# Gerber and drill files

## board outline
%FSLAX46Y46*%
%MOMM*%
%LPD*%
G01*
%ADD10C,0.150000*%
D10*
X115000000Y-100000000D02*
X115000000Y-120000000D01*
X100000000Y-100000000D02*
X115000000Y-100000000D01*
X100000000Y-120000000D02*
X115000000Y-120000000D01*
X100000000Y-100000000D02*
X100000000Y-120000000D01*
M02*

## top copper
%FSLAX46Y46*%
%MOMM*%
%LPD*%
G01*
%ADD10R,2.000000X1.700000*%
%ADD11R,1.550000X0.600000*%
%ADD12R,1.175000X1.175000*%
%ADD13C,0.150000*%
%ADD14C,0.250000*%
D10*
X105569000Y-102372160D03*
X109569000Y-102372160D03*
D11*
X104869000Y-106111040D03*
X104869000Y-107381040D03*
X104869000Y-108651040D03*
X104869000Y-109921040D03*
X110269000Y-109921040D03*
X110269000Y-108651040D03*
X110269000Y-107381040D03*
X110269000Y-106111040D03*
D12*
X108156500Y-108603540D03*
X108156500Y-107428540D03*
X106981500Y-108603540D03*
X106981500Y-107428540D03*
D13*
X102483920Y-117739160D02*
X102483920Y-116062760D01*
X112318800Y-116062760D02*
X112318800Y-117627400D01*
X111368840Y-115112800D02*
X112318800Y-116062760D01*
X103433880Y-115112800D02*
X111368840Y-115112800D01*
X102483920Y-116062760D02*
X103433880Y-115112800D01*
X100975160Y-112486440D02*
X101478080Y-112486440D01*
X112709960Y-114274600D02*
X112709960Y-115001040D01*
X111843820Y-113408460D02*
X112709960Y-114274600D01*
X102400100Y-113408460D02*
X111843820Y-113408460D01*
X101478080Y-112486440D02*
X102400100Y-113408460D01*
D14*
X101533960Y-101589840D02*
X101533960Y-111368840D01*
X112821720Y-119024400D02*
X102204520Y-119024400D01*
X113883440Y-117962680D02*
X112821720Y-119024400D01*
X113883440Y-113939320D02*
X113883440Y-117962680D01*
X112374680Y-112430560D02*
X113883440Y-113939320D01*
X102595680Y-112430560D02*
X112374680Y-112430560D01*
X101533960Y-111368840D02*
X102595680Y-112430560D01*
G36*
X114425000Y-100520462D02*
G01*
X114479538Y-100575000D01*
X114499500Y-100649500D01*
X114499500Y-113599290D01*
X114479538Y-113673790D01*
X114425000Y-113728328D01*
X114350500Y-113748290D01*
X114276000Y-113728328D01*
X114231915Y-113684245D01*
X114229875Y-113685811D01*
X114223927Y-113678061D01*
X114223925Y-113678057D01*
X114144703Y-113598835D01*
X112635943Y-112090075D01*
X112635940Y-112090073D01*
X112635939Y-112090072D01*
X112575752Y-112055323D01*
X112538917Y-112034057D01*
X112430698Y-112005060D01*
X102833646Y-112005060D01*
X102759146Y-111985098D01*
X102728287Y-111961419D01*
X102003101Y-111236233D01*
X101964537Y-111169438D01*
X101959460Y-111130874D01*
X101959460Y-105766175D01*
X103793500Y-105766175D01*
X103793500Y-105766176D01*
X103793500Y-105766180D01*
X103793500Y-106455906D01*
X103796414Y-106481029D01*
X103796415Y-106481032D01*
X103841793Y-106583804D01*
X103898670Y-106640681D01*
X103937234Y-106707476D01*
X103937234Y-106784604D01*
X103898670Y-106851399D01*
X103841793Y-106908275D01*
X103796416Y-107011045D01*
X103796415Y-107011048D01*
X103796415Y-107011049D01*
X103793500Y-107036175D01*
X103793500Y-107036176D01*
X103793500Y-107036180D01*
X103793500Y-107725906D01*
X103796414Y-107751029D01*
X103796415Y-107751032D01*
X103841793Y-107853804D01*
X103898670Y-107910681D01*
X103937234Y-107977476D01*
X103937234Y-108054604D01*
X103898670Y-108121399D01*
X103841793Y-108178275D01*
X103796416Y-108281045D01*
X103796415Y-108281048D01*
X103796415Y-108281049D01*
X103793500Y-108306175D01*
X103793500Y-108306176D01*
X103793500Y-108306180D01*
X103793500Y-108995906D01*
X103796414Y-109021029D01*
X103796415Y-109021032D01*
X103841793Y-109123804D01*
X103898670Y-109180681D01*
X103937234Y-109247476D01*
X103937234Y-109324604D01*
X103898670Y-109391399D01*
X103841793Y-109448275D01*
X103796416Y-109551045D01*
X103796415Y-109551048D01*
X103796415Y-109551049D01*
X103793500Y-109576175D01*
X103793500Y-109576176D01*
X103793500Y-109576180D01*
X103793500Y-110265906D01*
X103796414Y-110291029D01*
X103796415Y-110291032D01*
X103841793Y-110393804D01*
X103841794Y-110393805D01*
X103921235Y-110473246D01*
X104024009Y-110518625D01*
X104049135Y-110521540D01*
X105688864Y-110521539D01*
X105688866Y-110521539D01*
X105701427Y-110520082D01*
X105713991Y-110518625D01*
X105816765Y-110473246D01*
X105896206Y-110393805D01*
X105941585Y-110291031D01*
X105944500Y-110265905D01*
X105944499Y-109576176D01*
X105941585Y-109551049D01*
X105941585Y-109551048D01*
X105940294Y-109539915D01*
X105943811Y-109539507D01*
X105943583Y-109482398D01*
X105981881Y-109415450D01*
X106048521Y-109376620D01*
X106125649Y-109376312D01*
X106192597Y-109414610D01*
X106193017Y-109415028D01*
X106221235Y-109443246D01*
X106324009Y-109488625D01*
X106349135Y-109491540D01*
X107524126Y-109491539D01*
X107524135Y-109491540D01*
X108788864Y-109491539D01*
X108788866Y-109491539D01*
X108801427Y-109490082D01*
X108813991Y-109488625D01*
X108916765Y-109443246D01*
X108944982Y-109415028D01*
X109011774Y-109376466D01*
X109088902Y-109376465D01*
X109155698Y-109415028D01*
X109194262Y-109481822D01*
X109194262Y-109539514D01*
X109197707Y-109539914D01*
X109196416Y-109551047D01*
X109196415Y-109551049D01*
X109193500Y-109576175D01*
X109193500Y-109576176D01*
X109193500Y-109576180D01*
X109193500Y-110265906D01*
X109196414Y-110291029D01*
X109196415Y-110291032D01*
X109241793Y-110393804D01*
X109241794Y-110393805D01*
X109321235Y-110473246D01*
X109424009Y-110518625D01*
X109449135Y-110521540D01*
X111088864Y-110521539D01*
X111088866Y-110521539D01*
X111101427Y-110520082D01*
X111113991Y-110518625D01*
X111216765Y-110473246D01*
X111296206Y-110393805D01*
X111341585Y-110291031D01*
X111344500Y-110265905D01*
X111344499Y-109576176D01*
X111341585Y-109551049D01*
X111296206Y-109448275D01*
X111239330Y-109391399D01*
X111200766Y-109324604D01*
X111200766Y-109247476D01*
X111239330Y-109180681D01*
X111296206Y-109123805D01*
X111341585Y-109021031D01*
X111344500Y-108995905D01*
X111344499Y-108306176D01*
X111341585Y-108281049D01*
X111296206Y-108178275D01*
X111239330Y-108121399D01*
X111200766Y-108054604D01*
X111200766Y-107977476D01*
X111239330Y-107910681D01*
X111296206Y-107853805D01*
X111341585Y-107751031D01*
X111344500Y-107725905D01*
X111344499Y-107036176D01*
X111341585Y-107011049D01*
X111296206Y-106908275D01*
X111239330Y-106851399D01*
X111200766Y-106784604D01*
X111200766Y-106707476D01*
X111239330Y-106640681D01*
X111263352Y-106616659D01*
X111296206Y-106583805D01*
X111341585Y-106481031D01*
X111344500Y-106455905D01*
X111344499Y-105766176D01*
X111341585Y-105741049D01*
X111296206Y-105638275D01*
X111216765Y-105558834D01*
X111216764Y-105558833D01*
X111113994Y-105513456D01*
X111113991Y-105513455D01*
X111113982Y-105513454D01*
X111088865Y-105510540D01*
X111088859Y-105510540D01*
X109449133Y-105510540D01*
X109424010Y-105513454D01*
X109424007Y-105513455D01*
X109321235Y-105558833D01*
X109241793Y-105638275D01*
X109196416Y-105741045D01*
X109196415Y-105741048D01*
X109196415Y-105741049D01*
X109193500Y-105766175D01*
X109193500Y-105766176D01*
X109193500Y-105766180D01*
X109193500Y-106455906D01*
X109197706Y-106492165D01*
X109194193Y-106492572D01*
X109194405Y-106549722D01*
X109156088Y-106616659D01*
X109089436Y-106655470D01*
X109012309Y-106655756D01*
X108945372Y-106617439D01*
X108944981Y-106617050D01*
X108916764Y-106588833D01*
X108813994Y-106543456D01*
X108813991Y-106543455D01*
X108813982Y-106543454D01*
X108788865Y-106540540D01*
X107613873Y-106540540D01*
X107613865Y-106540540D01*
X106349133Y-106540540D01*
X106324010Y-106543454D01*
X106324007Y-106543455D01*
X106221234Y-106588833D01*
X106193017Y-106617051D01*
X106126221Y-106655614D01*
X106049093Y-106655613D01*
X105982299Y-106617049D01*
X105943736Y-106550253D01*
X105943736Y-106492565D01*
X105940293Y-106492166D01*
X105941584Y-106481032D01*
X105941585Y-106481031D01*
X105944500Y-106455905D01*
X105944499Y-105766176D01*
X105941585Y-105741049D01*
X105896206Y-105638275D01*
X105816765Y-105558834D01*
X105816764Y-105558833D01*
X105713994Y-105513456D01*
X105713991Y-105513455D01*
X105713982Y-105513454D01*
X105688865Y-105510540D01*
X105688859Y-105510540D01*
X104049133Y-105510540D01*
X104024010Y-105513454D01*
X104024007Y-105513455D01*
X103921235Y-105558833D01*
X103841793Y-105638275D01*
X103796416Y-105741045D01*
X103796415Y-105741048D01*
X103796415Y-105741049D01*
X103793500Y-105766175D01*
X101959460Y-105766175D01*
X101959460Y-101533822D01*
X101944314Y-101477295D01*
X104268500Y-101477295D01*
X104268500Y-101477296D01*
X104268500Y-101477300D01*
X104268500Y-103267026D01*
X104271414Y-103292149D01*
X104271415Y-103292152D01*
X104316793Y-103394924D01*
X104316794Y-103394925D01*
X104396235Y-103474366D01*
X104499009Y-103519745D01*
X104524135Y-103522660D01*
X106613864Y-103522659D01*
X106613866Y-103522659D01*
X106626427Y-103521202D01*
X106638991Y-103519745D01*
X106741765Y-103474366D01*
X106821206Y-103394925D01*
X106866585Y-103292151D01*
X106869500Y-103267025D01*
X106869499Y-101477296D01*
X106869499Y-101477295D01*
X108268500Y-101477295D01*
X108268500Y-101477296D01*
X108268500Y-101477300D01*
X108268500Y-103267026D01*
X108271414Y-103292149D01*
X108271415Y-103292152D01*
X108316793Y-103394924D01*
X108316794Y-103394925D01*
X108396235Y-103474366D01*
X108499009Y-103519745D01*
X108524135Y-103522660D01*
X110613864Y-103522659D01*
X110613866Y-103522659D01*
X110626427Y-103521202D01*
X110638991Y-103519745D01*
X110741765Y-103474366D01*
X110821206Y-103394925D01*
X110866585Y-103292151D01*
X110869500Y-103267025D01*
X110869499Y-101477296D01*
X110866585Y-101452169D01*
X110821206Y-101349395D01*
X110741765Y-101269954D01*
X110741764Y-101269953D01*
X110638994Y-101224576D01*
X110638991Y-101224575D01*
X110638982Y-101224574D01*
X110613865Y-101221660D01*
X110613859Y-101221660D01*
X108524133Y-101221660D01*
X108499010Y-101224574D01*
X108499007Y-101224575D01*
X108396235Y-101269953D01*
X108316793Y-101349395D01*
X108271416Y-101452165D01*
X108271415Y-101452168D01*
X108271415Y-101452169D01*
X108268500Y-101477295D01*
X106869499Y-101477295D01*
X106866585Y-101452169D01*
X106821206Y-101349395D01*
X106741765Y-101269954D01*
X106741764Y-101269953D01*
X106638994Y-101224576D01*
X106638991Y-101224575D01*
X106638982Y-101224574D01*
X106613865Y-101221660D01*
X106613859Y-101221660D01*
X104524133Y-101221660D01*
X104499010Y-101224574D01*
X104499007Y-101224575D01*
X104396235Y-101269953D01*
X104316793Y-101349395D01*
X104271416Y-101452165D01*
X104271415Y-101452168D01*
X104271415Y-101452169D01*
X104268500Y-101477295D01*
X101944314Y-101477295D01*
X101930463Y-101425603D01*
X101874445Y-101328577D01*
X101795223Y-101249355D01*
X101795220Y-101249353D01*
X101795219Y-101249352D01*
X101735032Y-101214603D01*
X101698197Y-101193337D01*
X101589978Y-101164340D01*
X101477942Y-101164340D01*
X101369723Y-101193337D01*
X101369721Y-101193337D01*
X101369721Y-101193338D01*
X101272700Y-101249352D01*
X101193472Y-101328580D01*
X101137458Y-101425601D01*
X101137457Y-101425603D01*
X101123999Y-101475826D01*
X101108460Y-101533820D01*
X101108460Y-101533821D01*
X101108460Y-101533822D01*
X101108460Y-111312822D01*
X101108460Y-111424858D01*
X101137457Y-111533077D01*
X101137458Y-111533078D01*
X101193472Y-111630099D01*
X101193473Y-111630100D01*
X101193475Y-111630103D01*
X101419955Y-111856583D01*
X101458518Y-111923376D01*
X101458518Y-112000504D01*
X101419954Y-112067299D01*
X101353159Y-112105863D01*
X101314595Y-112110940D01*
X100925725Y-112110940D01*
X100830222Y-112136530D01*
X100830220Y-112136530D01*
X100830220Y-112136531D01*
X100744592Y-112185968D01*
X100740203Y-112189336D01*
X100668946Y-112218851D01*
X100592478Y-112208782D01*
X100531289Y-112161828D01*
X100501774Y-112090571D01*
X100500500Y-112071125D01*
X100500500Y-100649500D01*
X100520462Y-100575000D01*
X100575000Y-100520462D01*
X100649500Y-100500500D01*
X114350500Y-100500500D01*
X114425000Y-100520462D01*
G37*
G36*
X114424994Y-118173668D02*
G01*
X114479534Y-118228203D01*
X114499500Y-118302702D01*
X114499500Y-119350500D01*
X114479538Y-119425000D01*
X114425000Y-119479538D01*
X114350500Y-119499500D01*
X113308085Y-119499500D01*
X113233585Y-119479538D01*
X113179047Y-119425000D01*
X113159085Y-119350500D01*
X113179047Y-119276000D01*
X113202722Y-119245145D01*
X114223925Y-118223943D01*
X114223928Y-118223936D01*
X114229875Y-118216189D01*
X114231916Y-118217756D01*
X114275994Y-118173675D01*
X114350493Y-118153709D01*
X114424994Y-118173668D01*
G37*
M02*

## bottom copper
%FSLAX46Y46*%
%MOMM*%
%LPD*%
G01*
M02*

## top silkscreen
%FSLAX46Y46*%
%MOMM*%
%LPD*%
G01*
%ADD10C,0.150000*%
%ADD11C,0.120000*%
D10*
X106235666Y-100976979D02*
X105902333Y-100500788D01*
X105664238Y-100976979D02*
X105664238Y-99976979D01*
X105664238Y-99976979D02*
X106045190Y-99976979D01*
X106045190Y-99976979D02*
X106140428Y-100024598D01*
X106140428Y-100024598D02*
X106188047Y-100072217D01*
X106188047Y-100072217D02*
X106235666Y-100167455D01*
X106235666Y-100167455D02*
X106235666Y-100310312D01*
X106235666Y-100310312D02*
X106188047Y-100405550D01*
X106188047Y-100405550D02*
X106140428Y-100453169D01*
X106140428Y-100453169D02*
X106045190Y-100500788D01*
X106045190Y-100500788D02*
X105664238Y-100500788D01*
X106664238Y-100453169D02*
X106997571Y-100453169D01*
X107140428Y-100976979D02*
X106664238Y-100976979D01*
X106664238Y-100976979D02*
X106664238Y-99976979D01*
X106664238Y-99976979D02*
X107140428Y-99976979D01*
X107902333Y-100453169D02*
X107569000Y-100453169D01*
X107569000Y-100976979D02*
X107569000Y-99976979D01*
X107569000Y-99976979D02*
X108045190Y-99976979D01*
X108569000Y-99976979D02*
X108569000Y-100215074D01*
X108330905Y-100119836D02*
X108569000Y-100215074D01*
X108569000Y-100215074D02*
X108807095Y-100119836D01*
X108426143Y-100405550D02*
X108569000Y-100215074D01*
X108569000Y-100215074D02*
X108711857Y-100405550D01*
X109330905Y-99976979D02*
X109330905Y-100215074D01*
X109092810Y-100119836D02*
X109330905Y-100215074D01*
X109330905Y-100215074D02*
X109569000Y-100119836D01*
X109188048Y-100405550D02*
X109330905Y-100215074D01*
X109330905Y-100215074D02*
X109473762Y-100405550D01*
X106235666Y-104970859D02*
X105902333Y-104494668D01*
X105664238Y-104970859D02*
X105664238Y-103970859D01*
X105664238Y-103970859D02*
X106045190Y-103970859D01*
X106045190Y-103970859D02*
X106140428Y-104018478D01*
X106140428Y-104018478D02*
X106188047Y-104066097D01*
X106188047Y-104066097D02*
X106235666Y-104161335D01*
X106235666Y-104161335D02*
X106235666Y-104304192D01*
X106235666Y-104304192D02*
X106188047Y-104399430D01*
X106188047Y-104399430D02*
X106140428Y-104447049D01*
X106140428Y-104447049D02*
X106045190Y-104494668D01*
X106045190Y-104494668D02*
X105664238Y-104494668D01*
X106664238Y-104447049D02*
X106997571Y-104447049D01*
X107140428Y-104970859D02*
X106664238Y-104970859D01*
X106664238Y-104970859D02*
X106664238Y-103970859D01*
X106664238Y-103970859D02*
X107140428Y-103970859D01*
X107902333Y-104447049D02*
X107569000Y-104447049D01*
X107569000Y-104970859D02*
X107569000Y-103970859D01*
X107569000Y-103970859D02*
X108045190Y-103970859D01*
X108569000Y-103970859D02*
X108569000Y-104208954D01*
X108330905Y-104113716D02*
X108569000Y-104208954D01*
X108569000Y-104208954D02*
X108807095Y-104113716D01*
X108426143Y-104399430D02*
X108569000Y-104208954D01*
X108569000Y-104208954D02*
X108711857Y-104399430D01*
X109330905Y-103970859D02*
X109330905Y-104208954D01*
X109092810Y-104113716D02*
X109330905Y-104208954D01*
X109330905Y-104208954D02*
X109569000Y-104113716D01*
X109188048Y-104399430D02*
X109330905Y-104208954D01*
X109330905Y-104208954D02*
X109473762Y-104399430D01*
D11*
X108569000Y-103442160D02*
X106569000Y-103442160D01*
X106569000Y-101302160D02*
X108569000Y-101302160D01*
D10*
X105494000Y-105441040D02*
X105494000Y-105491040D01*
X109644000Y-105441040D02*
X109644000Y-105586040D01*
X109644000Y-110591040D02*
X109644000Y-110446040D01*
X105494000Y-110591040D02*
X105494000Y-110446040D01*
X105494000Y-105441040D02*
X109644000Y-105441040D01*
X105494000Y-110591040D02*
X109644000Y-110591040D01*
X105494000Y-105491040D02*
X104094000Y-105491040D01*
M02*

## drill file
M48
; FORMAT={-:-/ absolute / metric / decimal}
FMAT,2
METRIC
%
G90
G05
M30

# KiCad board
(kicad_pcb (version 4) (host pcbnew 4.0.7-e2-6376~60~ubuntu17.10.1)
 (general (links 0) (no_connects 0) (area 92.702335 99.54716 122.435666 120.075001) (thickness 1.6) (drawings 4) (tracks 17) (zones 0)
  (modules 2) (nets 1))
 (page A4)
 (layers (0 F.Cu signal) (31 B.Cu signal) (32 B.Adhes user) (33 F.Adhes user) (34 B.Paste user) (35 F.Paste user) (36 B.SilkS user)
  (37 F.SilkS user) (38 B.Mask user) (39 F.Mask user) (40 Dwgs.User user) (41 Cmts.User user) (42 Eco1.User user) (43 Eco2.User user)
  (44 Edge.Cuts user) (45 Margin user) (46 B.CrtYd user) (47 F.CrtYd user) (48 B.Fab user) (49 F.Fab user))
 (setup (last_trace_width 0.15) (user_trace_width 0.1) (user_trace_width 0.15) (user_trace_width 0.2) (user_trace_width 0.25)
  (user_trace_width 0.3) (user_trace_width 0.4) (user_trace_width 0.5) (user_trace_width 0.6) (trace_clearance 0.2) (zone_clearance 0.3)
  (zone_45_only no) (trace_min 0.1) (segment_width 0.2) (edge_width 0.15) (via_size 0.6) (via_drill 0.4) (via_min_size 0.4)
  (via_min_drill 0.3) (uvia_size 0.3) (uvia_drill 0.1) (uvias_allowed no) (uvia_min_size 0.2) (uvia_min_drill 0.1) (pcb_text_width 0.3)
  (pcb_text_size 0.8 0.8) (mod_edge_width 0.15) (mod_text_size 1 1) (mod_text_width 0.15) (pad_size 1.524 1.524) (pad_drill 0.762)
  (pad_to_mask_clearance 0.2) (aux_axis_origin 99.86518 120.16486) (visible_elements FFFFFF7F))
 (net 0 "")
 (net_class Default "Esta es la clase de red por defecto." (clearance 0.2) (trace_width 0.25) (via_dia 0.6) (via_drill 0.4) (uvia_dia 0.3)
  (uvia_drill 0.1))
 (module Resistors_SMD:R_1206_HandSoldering (layer F.Cu) (at 107.569 102.37216)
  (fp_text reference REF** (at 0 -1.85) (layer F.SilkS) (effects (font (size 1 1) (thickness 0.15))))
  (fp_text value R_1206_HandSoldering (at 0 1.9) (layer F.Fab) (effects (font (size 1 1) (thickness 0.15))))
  (fp_line (start 1 1.07) (end -1 1.07) (layer F.SilkS) (width 0.12))
  (fp_line (start -1 -1.07) (end 1 -1.07) (layer F.SilkS) (width 0.12))
  (pad 1 smd rect (at -2 0) (size 2 1.7) (layers F.Cu F.Paste F.Mask))
  (pad 2 smd rect (at 2 0) (size 2 1.7) (layers F.Cu F.Paste F.Mask)))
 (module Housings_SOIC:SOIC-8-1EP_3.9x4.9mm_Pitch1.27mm (layer F.Cu) (at 107.569 108.01604)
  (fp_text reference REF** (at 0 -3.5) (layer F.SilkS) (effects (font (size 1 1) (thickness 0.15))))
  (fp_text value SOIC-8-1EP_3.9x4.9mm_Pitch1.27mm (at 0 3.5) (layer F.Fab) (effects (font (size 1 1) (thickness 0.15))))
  (fp_line (start -2.075 -2.575) (end -2.075 -2.525) (layer F.SilkS) (width 0.15))
  (fp_line (start 2.075 -2.575) (end 2.075 -2.43) (layer F.SilkS) (width 0.15))
  (fp_line (start 2.075 2.575) (end 2.075 2.43) (layer F.SilkS) (width 0.15))
  (fp_line (start -2.075 2.575) (end -2.075 2.43) (layer F.SilkS) (width 0.15))
  (fp_line (start -2.075 -2.575) (end 2.075 -2.575) (layer F.SilkS) (width 0.15))
  (fp_line (start -2.075 2.575) (end 2.075 2.575) (layer F.SilkS) (width 0.15))
  (fp_line (start -2.075 -2.525) (end -3.475 -2.525) (layer F.SilkS) (width 0.15))
  (pad 1 smd rect (at -2.7 -1.905) (size 1.55 0.6) (layers F.Cu F.Paste F.Mask))
  (pad 2 smd rect (at -2.7 -0.635) (size 1.55 0.6) (layers F.Cu F.Paste F.Mask))
  (pad 3 smd rect (at -2.7 0.635) (size 1.55 0.6) (layers F.Cu F.Paste F.Mask))
  (pad 4 smd rect (at -2.7 1.905) (size 1.55 0.6) (layers F.Cu F.Paste F.Mask))
  (pad 5 smd rect (at 2.7 1.905) (size 1.55 0.6) (layers F.Cu F.Paste F.Mask))
  (pad 6 smd rect (at 2.7 0.635) (size 1.55 0.6) (layers F.Cu F.Paste F.Mask))
  (pad 7 smd rect (at 2.7 -0.635) (size 1.55 0.6) (layers F.Cu F.Paste F.Mask))
  (pad 8 smd rect (at 2.7 -1.905) (size 1.55 0.6) (layers F.Cu F.Paste F.Mask))
  (pad 9 smd rect (at 0.5875 0.5875) (size 1.175 1.175) (layers F.Cu F.Paste F.Mask) (solder_paste_margin_ratio -0.2))
  (pad 9 smd rect (at 0.5875 -0.5875) (size 1.175 1.175) (layers F.Cu F.Paste F.Mask) (solder_paste_margin_ratio -0.2))
  (pad 9 smd rect (at -0.5875 0.5875) (size 1.175 1.175) (layers F.Cu F.Paste F.Mask) (solder_paste_margin_ratio -0.2))
  (pad 9 smd rect (at -0.5875 -0.5875) (size 1.175 1.175) (layers F.Cu F.Paste F.Mask) (solder_paste_margin_ratio -0.2)))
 (gr_line (start 115 100) (end 115 120) (angle 90) (layer Edge.Cuts) (width 0.15))
 (gr_line (start 100 100) (end 115 100) (angle 90) (layer Edge.Cuts) (width 0.15))
 (gr_line (start 100 120) (end 115 120) (angle 90) (layer Edge.Cuts) (width 0.15))
 (gr_line (start 100 100) (end 100 120) (angle 90) (layer Edge.Cuts) (width 0.15))
 (segment (start 102.48392 117.73916) (end 102.48392 116.06276) (width 0.15) (layer F.Cu) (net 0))
 (segment (start 112.3188 116.06276) (end 112.3188 117.6274) (width 0.15) (layer F.Cu) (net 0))
 (segment (start 111.36884 115.1128) (end 112.3188 116.06276) (width 0.15) (layer F.Cu) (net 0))
 (segment (start 103.43388 115.1128) (end 111.36884 115.1128) (width 0.15) (layer F.Cu) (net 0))
 (segment (start 102.48392 116.06276) (end 103.43388 115.1128) (width 0.15) (layer F.Cu) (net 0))
 (segment (start 100.97516 112.48644) (end 101.47808 112.48644) (width 0.15) (layer F.Cu) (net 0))
 (segment (start 112.70996 114.2746) (end 112.70996 115.00104) (width 0.15) (layer F.Cu) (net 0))
 (segment (start 111.84382 113.40846) (end 112.70996 114.2746) (width 0.15) (layer F.Cu) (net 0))
 (segment (start 102.4001 113.40846) (end 111.84382 113.40846) (width 0.15) (layer F.Cu) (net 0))
 (segment (start 101.47808 112.48644) (end 102.4001 113.40846) (width 0.15) (layer F.Cu) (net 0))
 (segment (start 101.53396 101.58984) (end 101.53396 111.36884) (width 0.25) (layer F.Cu) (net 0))
 (segment (start 112.82172 119.0244) (end 102.20452 119.0244) (width 0.25) (layer F.Cu) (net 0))
 (segment (start 113.88344 117.96268) (end 112.82172 119.0244) (width 0.25) (layer F.Cu) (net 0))
 (segment (start 113.88344 113.93932) (end 113.88344 117.96268) (width 0.25) (layer F.Cu) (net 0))
 (segment (start 112.37468 112.43056) (end 113.88344 113.93932) (width 0.25) (layer F.Cu) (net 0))
 (segment (start 102.59568 112.43056) (end 112.37468 112.43056) (width 0.25) (layer F.Cu) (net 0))
 (segment (start 101.53396 111.36884) (end 102.59568 112.43056) (width 0.25) (layer F.Cu) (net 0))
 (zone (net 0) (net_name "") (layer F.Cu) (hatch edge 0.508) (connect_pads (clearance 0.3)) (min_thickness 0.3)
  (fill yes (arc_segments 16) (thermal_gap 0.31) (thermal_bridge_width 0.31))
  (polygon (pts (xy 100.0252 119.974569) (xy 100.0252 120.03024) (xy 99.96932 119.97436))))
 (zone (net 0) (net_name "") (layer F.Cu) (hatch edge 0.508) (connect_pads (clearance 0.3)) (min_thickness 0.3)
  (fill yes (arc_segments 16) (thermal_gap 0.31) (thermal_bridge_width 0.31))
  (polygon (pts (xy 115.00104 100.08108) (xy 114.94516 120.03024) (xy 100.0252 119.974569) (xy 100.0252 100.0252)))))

